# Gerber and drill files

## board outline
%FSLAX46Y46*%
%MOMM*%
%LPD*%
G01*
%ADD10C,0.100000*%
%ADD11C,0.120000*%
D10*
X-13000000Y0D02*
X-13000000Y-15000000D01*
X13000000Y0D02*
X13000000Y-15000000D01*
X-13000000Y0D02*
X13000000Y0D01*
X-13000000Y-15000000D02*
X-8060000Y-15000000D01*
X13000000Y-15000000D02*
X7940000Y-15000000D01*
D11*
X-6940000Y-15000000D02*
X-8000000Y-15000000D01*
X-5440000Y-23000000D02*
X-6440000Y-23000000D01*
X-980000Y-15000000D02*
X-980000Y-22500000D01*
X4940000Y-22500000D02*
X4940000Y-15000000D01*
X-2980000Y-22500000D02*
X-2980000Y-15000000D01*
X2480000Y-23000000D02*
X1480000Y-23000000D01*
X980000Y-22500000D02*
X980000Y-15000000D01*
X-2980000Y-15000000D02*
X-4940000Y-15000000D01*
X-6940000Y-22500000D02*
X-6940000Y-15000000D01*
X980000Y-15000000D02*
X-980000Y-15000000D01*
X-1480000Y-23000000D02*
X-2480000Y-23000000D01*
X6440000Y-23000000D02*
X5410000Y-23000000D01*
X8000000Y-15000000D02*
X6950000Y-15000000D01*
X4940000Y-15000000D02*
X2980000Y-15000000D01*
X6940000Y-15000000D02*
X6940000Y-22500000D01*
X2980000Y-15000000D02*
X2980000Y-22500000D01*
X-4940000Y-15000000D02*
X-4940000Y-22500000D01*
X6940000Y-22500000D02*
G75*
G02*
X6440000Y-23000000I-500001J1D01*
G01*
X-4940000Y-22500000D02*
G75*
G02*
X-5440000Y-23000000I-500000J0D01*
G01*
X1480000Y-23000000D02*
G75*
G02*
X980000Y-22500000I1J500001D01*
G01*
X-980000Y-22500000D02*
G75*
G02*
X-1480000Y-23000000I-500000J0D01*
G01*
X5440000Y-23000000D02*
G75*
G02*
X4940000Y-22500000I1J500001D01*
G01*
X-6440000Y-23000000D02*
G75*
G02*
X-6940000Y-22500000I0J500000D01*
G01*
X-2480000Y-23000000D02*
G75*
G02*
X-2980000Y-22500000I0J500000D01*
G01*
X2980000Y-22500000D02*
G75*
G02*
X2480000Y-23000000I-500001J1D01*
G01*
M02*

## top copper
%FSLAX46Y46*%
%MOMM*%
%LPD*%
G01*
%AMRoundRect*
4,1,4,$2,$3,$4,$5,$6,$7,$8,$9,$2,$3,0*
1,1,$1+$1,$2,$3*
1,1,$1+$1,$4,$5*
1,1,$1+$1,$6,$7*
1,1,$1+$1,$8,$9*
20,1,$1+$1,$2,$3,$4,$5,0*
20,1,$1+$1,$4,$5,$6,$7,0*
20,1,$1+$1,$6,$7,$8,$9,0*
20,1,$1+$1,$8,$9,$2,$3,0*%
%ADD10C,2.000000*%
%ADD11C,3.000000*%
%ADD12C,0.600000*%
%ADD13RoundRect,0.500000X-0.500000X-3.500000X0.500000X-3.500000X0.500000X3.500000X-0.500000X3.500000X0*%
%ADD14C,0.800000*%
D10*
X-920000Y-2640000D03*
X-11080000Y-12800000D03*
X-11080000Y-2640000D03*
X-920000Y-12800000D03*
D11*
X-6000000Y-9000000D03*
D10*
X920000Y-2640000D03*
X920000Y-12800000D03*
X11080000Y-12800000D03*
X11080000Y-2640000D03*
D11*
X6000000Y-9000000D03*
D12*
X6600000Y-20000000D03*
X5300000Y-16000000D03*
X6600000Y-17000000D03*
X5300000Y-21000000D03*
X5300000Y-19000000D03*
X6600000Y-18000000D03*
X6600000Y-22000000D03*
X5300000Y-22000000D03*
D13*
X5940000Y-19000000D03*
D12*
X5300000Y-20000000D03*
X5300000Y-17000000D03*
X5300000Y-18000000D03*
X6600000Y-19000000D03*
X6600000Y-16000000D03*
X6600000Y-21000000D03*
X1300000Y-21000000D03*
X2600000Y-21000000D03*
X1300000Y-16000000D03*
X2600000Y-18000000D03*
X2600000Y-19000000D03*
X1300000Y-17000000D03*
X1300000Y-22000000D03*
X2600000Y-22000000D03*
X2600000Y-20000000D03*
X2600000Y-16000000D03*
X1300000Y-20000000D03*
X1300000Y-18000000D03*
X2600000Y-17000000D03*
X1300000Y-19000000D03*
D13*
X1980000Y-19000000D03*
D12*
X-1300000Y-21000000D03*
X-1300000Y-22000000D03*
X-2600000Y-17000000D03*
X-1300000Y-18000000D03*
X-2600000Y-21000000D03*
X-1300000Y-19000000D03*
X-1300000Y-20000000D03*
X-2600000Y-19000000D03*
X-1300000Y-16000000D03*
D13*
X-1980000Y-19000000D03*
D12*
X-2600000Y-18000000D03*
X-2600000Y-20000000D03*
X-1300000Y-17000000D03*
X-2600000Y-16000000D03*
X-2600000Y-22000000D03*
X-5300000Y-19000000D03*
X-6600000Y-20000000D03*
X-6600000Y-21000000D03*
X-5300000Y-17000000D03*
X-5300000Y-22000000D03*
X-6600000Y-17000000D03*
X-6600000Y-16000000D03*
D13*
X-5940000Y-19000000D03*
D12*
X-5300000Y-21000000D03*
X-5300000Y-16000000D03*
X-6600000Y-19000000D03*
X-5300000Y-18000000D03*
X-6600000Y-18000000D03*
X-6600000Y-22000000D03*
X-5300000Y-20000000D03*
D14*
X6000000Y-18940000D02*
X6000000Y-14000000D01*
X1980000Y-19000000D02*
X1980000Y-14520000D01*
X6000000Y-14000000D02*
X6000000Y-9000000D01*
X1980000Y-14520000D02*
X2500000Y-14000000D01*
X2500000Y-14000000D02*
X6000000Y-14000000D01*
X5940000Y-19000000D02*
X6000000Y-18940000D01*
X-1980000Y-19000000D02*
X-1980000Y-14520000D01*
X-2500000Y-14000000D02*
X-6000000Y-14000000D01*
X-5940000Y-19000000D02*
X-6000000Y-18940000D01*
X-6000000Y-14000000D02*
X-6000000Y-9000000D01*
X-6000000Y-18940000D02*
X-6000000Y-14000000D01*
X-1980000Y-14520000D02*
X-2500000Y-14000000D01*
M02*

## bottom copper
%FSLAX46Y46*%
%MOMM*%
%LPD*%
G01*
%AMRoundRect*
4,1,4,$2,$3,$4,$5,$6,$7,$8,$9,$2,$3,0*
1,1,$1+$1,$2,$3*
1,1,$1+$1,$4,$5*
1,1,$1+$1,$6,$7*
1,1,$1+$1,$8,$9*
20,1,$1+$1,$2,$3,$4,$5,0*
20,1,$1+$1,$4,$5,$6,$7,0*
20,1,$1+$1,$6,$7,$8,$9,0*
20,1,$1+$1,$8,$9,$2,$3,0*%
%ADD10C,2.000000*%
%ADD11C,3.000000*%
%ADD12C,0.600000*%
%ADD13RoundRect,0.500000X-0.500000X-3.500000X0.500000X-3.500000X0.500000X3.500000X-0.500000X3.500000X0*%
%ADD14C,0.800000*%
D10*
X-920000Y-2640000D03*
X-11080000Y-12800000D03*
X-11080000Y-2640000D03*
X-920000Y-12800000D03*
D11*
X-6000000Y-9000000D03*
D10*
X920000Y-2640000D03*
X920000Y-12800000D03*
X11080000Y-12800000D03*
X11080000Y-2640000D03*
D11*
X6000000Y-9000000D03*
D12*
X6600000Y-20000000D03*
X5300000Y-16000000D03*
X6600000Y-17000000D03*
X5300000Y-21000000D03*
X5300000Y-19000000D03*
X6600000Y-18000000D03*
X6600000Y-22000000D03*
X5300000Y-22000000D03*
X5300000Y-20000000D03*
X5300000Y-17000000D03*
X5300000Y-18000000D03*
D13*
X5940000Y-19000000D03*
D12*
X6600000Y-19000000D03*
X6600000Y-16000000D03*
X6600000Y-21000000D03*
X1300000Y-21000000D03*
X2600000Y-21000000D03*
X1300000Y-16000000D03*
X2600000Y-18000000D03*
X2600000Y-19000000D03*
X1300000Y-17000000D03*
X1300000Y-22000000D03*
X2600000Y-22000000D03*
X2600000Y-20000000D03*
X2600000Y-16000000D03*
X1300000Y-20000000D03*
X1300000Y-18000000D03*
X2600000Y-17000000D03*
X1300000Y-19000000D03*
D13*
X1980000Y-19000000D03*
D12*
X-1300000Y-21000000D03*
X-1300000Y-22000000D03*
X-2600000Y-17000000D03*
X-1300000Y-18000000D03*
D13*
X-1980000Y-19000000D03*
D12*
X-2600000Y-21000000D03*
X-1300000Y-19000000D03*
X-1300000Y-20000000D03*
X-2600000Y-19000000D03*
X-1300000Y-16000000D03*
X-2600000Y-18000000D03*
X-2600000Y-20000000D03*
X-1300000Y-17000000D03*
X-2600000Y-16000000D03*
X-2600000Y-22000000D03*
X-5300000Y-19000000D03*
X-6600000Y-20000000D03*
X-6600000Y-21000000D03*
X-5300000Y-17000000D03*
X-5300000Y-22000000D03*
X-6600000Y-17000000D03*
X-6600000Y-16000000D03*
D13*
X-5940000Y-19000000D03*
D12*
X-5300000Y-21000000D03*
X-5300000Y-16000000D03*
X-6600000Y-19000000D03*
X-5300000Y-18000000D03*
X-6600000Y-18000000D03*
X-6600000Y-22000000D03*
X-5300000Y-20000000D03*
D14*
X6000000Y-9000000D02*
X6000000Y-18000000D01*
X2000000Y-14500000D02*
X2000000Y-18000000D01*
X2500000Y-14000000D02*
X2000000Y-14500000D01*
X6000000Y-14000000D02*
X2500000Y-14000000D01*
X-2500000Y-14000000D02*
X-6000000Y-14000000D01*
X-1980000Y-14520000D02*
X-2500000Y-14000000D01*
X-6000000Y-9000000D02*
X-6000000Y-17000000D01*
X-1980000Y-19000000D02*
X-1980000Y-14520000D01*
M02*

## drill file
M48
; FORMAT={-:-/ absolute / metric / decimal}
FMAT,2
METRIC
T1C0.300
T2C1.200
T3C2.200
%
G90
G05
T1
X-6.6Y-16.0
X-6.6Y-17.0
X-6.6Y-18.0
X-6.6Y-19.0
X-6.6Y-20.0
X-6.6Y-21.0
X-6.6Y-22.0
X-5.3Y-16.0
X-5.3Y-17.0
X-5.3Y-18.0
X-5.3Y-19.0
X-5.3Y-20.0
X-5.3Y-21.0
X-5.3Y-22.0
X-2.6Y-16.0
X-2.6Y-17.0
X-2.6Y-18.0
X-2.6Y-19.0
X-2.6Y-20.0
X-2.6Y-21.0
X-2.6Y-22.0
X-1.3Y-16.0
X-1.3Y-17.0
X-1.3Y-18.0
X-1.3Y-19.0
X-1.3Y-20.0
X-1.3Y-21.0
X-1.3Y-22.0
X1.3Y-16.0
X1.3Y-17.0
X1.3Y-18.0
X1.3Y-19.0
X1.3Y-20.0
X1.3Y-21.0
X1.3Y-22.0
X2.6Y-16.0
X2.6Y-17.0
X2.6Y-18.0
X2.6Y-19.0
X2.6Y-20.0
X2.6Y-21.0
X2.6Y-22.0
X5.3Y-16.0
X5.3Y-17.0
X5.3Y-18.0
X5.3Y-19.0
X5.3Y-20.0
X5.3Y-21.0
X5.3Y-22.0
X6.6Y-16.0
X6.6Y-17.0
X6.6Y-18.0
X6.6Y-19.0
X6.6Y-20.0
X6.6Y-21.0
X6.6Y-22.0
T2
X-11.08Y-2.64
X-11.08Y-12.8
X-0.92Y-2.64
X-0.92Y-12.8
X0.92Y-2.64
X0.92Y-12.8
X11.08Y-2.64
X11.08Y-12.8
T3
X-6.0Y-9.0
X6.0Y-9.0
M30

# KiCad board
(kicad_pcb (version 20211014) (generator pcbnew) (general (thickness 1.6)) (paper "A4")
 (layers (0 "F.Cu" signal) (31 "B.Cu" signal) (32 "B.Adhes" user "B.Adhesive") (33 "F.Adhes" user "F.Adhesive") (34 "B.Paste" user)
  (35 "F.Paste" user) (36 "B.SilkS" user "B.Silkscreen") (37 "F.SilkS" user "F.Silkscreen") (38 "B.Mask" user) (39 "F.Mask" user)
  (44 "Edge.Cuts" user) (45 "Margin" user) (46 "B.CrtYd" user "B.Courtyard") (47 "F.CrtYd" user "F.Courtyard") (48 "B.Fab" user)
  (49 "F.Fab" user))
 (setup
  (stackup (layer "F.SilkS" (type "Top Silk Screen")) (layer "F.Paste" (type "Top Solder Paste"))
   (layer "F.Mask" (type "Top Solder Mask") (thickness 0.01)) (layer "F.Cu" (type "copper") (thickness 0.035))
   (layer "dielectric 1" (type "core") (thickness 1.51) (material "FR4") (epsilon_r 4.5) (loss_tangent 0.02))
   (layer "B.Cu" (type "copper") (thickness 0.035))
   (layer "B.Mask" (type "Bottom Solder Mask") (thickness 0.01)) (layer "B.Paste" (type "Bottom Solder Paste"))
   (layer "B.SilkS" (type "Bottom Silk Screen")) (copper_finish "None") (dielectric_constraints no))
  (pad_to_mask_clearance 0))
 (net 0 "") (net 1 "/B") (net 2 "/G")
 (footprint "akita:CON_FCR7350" (layer "F.Cu") (at -6 9 -90)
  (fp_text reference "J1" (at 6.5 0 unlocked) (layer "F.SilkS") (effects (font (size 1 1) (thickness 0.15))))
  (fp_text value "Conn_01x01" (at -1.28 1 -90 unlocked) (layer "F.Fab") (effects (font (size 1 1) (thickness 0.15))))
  (pad "-" thru_hole circle (at -6.36 -5.08 270) (size 2 2) (drill 1.2) (layers *.Cu *.Mask))
  (pad "-" thru_hole circle (at 3.8 5.08 270) (size 2 2) (drill 1.2) (layers *.Cu *.Mask))
  (pad "-" thru_hole circle (at -6.36 5.08 270) (size 2 2) (drill 1.2) (layers *.Cu *.Mask))
  (pad "-" thru_hole circle (at 3.8 -5.08 270) (size 2 2) (drill 1.2) (layers *.Cu *.Mask))
  (pad "1" thru_hole circle (at 0 0 270) (size 3 3) (drill 2.2) (layers *.Cu *.Mask) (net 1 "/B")))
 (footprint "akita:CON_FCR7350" (layer "F.Cu") (at 6 9 -90)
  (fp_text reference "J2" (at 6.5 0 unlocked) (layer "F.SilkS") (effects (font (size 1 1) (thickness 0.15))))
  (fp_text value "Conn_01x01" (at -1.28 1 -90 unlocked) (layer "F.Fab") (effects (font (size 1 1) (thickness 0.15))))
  (pad "-" thru_hole circle (at -6.36 5.08 270) (size 2 2) (drill 1.2) (layers *.Cu *.Mask))
  (pad "-" thru_hole circle (at 3.8 5.08 270) (size 2 2) (drill 1.2) (layers *.Cu *.Mask))
  (pad "-" thru_hole circle (at 3.8 -5.08 270) (size 2 2) (drill 1.2) (layers *.Cu *.Mask))
  (pad "-" thru_hole circle (at -6.36 -5.08 270) (size 2 2) (drill 1.2) (layers *.Cu *.Mask))
  (pad "1" thru_hole circle (at 0 0 270) (size 3 3) (drill 2.2) (layers *.Cu *.Mask) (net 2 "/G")))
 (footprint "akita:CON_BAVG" (layer "F.Cu") (at 0 19 180)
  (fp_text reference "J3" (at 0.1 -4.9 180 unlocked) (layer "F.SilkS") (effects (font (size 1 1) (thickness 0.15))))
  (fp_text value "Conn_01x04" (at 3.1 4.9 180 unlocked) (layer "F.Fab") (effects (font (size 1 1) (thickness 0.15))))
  (fp_line (start 6.94 4) (end 8 4) (layer "Edge.Cuts") (width 0.12))
  (fp_line (start 5.44 -4) (end 6.44 -4) (layer "Edge.Cuts") (width 0.12))
  (fp_line (start 0.98 4) (end 0.98 -3.5) (layer "Edge.Cuts") (width 0.12))
  (fp_line (start -4.94 -3.5) (end -4.94 4) (layer "Edge.Cuts") (width 0.12))
  (fp_line (start 2.98 -3.5) (end 2.98 4) (layer "Edge.Cuts") (width 0.12))
  (fp_line (start -2.48 -4) (end -1.48 -4) (layer "Edge.Cuts") (width 0.12))
  (fp_line (start -0.98 -3.5) (end -0.98 4) (layer "Edge.Cuts") (width 0.12))
  (fp_line (start 2.98 4) (end 4.94 4) (layer "Edge.Cuts") (width 0.12))
  (fp_line (start 6.94 -3.5) (end 6.94 4) (layer "Edge.Cuts") (width 0.12))
  (fp_line (start -0.98 4) (end 0.98 4) (layer "Edge.Cuts") (width 0.12))
  (fp_line (start 1.48 -4) (end 2.48 -4) (layer "Edge.Cuts") (width 0.12))
  (fp_line (start -6.44 -4) (end -5.41 -4) (layer "Edge.Cuts") (width 0.12))
  (fp_line (start -8 4) (end -6.95 4) (layer "Edge.Cuts") (width 0.12))
  (fp_line (start -4.94 4) (end -2.98 4) (layer "Edge.Cuts") (width 0.12))
  (fp_line (start -6.94 4) (end -6.94 -3.5) (layer "Edge.Cuts") (width 0.12))
  (fp_line (start -2.98 4) (end -2.98 -3.5) (layer "Edge.Cuts") (width 0.12))
  (fp_line (start 4.94 4) (end 4.94 -3.5) (layer "Edge.Cuts") (width 0.12))
  (fp_arc (start -6.94 -3.5) (mid -6.793553 -3.853553) (end -6.44 -4) (layer "Edge.Cuts") (width 0.12))
  (fp_arc (start 4.94 -3.5) (mid 5.086447 -3.853553) (end 5.44 -4) (layer "Edge.Cuts") (width 0.12))
  (fp_arc (start -1.48 -4) (mid -1.126447 -3.853553) (end -0.98 -3.5) (layer "Edge.Cuts") (width 0.12))
  (fp_arc (start 0.98 -3.5) (mid 1.126447 -3.853553) (end 1.48 -4) (layer "Edge.Cuts") (width 0.12))
  (fp_arc (start -5.44 -4) (mid -5.086447 -3.853553) (end -4.94 -3.5) (layer "Edge.Cuts") (width 0.12))
  (fp_arc (start 6.44 -4) (mid 6.793553 -3.853553) (end 6.94 -3.5) (layer "Edge.Cuts") (width 0.12))
  (fp_arc (start 2.48 -4) (mid 2.833553 -3.853553) (end 2.98 -3.5) (layer "Edge.Cuts") (width 0.12))
  (fp_arc (start -2.98 -3.5) (mid -2.833553 -3.853553) (end -2.48 -4) (layer "Edge.Cuts") (width 0.12))
  (pad "1" thru_hole circle (at -6.6 -1 180) (size 0.6 0.6) (drill 0.3) (layers *.Cu *.Mask) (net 2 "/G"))
  (pad "1" thru_hole circle (at -5.3 3 180) (size 0.6 0.6) (drill 0.3) (layers *.Cu *.Mask) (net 2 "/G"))
  (pad "1" thru_hole circle (at -6.6 2 180) (size 0.6 0.6) (drill 0.3) (layers *.Cu *.Mask) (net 2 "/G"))
  (pad "1" thru_hole circle (at -5.3 -2 180) (size 0.6 0.6) (drill 0.3) (layers *.Cu *.Mask) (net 2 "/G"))
  (pad "1" thru_hole circle (at -5.3 0 180) (size 0.6 0.6) (drill 0.3) (layers *.Cu *.Mask) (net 2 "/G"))
  (pad "1" thru_hole circle (at -6.6 1 180) (size 0.6 0.6) (drill 0.3) (layers *.Cu *.Mask) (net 2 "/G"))
  (pad "1" thru_hole circle (at -6.6 -3 180) (size 0.6 0.6) (drill 0.3) (layers *.Cu *.Mask) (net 2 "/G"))
  (pad "1" thru_hole circle (at -5.3 -3 180) (size 0.6 0.6) (drill 0.3) (layers *.Cu *.Mask) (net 2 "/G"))
  (pad "1" smd roundrect (at -5.94 0) (size 2 8) (layers "F.Cu" "F.Paste" "F.Mask") (roundrect_rratio 0.25) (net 2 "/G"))
  (pad "1" thru_hole circle (at -5.3 -1 180) (size 0.6 0.6) (drill 0.3) (layers *.Cu *.Mask) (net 2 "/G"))
  (pad "1" thru_hole circle (at -5.3 2 180) (size 0.6 0.6) (drill 0.3) (layers *.Cu *.Mask) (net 2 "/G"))
  (pad "1" thru_hole circle (at -5.3 1 180) (size 0.6 0.6) (drill 0.3) (layers *.Cu *.Mask) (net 2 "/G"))
  (pad "1" smd roundrect (at -5.94 0) (size 2 8) (layers "B.Cu" "B.Paste" "B.Mask") (roundrect_rratio 0.25) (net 2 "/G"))
  (pad "1" thru_hole circle (at -6.6 0 180) (size 0.6 0.6) (drill 0.3) (layers *.Cu *.Mask) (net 2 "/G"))
  (pad "1" thru_hole circle (at -6.6 3 180) (size 0.6 0.6) (drill 0.3) (layers *.Cu *.Mask) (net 2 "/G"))
  (pad "1" thru_hole circle (at -6.6 -2 180) (size 0.6 0.6) (drill 0.3) (layers *.Cu *.Mask) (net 2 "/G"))
  (pad "2" thru_hole circle (at -1.3 -2 180) (size 0.6 0.6) (drill 0.3) (layers *.Cu *.Mask) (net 2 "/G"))
  (pad "2" thru_hole circle (at -2.6 -2 180) (size 0.6 0.6) (drill 0.3) (layers *.Cu *.Mask) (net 2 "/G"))
  (pad "2" thru_hole circle (at -1.3 3 180) (size 0.6 0.6) (drill 0.3) (layers *.Cu *.Mask) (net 2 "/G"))
  (pad "2" thru_hole circle (at -2.6 1 180) (size 0.6 0.6) (drill 0.3) (layers *.Cu *.Mask) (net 2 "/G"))
  (pad "2" thru_hole circle (at -2.6 0 180) (size 0.6 0.6) (drill 0.3) (layers *.Cu *.Mask) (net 2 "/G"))
  (pad "2" thru_hole circle (at -1.3 2 180) (size 0.6 0.6) (drill 0.3) (layers *.Cu *.Mask) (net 2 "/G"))
  (pad "2" thru_hole circle (at -1.3 -3 180) (size 0.6 0.6) (drill 0.3) (layers *.Cu *.Mask) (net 2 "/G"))
  (pad "2" thru_hole circle (at -2.6 -3 180) (size 0.6 0.6) (drill 0.3) (layers *.Cu *.Mask) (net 2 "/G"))
  (pad "2" thru_hole circle (at -2.6 -1 180) (size 0.6 0.6) (drill 0.3) (layers *.Cu *.Mask) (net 2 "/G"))
  (pad "2" thru_hole circle (at -2.6 3 180) (size 0.6 0.6) (drill 0.3) (layers *.Cu *.Mask) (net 2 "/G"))
  (pad "2" thru_hole circle (at -1.3 -1 180) (size 0.6 0.6) (drill 0.3) (layers *.Cu *.Mask) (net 2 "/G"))
  (pad "2" thru_hole circle (at -1.3 1 180) (size 0.6 0.6) (drill 0.3) (layers *.Cu *.Mask) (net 2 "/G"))
  (pad "2" thru_hole circle (at -2.6 2 180) (size 0.6 0.6) (drill 0.3) (layers *.Cu *.Mask) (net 2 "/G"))
  (pad "2" thru_hole circle (at -1.3 0 180) (size 0.6 0.6) (drill 0.3) (layers *.Cu *.Mask) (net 2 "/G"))
  (pad "2" smd roundrect (at -1.98 0) (size 2 8) (layers "F.Cu" "F.Paste" "F.Mask") (roundrect_rratio 0.25) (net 2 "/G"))
  (pad "2" smd roundrect (at -1.98 0) (size 2 8) (layers "B.Cu" "B.Paste" "B.Mask") (roundrect_rratio 0.25) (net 2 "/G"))
  (pad "3" thru_hole circle (at 1.3 -2 180) (size 0.6 0.6) (drill 0.3) (layers *.Cu *.Mask) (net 1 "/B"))
  (pad "3" thru_hole circle (at 1.3 -3 180) (size 0.6 0.6) (drill 0.3) (layers *.Cu *.Mask) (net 1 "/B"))
  (pad "3" thru_hole circle (at 2.6 2 180) (size 0.6 0.6) (drill 0.3) (layers *.Cu *.Mask) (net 1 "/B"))
  (pad "3" thru_hole circle (at 1.3 1 180) (size 0.6 0.6) (drill 0.3) (layers *.Cu *.Mask) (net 1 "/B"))
  (pad "3" smd roundrect (at 1.98 0) (size 2 8) (layers "B.Cu" "B.Paste" "B.Mask") (roundrect_rratio 0.25) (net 1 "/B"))
  (pad "3" thru_hole circle (at 2.6 -2 180) (size 0.6 0.6) (drill 0.3) (layers *.Cu *.Mask) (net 1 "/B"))
  (pad "3" thru_hole circle (at 1.3 0 180) (size 0.6 0.6) (drill 0.3) (layers *.Cu *.Mask) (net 1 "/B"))
  (pad "3" thru_hole circle (at 1.3 -1 180) (size 0.6 0.6) (drill 0.3) (layers *.Cu *.Mask) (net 1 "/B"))
  (pad "3" thru_hole circle (at 2.6 0 180) (size 0.6 0.6) (drill 0.3) (layers *.Cu *.Mask) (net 1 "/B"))
  (pad "3" thru_hole circle (at 1.3 3 180) (size 0.6 0.6) (drill 0.3) (layers *.Cu *.Mask) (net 1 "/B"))
  (pad "3" smd roundrect (at 1.98 0) (size 2 8) (layers "F.Cu" "F.Paste" "F.Mask") (roundrect_rratio 0.25) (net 1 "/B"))
  (pad "3" thru_hole circle (at 2.6 1 180) (size 0.6 0.6) (drill 0.3) (layers *.Cu *.Mask) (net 1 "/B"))
  (pad "3" thru_hole circle (at 2.6 -1 180) (size 0.6 0.6) (drill 0.3) (layers *.Cu *.Mask) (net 1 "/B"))
  (pad "3" thru_hole circle (at 1.3 2 180) (size 0.6 0.6) (drill 0.3) (layers *.Cu *.Mask) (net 1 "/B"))
  (pad "3" thru_hole circle (at 2.6 3 180) (size 0.6 0.6) (drill 0.3) (layers *.Cu *.Mask) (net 1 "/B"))
  (pad "3" thru_hole circle (at 2.6 -3 180) (size 0.6 0.6) (drill 0.3) (layers *.Cu *.Mask) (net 1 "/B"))
  (pad "4" thru_hole circle (at 5.3 0 180) (size 0.6 0.6) (drill 0.3) (layers *.Cu *.Mask) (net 1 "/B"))
  (pad "4" thru_hole circle (at 6.6 -1 180) (size 0.6 0.6) (drill 0.3) (layers *.Cu *.Mask) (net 1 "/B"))
  (pad "4" thru_hole circle (at 6.6 -2 180) (size 0.6 0.6) (drill 0.3) (layers *.Cu *.Mask) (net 1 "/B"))
  (pad "4" thru_hole circle (at 5.3 2 180) (size 0.6 0.6) (drill 0.3) (layers *.Cu *.Mask) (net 1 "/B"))
  (pad "4" thru_hole circle (at 5.3 -3 180) (size 0.6 0.6) (drill 0.3) (layers *.Cu *.Mask) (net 1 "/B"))
  (pad "4" thru_hole circle (at 6.6 2 180) (size 0.6 0.6) (drill 0.3) (layers *.Cu *.Mask) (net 1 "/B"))
  (pad "4" thru_hole circle (at 6.6 3 180) (size 0.6 0.6) (drill 0.3) (layers *.Cu *.Mask) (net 1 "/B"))
  (pad "4" smd roundrect (at 5.94 0) (size 2 8) (layers "F.Cu" "F.Paste" "F.Mask") (roundrect_rratio 0.25) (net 1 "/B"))
  (pad "4" smd roundrect (at 5.94 0) (size 2 8) (layers "B.Cu" "B.Paste" "B.Mask") (roundrect_rratio 0.25) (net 1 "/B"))
  (pad "4" thru_hole circle (at 5.3 -2 180) (size 0.6 0.6) (drill 0.3) (layers *.Cu *.Mask) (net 1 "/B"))
  (pad "4" thru_hole circle (at 5.3 3 180) (size 0.6 0.6) (drill 0.3) (layers *.Cu *.Mask) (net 1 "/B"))
  (pad "4" thru_hole circle (at 6.6 0 180) (size 0.6 0.6) (drill 0.3) (layers *.Cu *.Mask) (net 1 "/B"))
  (pad "4" thru_hole circle (at 5.3 1 180) (size 0.6 0.6) (drill 0.3) (layers *.Cu *.Mask) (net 1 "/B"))
  (pad "4" thru_hole circle (at 6.6 1 180) (size 0.6 0.6) (drill 0.3) (layers *.Cu *.Mask) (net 1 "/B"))
  (pad "4" thru_hole circle (at 6.6 -3 180) (size 0.6 0.6) (drill 0.3) (layers *.Cu *.Mask) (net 1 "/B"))
  (pad "4" thru_hole circle (at 5.3 -1 180) (size 0.6 0.6) (drill 0.3) (layers *.Cu *.Mask) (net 1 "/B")))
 (gr_line (start -13 0) (end -13 15) (layer "Edge.Cuts") (width 0.1))
 (gr_line (start 13 0) (end 13 15) (layer "Edge.Cuts") (width 0.1))
 (gr_line (start -13 0) (end 13 0) (layer "Edge.Cuts") (width 0.1))
 (gr_line (start -13 15) (end -8.06 15) (layer "Edge.Cuts") (width 0.1))
 (gr_line (start 13 15) (end 7.94 15) (layer "Edge.Cuts") (width 0.1))
 (segment (start 6 18.94) (end 6 14) (width 0.8) (layer "F.Cu") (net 2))
 (segment (start 1.98 19) (end 1.98 14.52) (width 0.8) (layer "F.Cu") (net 2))
 (segment (start 6 14) (end 6 9) (width 0.8) (layer "F.Cu") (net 2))
 (segment (start 1.98 14.52) (end 2.5 14) (width 0.8) (layer "F.Cu") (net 2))
 (segment (start 2.5 14) (end 6 14) (width 0.8) (layer "F.Cu") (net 2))
 (segment (start 5.94 19) (end 6 18.94) (width 0.8) (layer "F.Cu") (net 2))
 (segment (start 6 9) (end 6 18) (width 0.8) (layer "B.Cu") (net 2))
 (segment (start 2 14.5) (end 2 18) (width 0.8) (layer "B.Cu") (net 2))
 (segment (start 2.5 14) (end 2 14.5) (width 0.8) (layer "B.Cu") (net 2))
 (segment (start 6 14) (end 2.5 14) (width 0.8) (layer "B.Cu") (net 2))
 (segment (start -1.98 19) (end -1.98 14.52) (width 0.8) (layer "F.Cu") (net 1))
 (segment (start -2.5 14) (end -6 14) (width 0.8) (layer "F.Cu") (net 1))
 (segment (start -5.94 19) (end -6 18.94) (width 0.8) (layer "F.Cu") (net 1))
 (segment (start -6 14) (end -6 9) (width 0.8) (layer "F.Cu") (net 1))
 (segment (start -6 18.94) (end -6 14) (width 0.8) (layer "F.Cu") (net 1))
 (segment (start -1.98 14.52) (end -2.5 14) (width 0.8) (layer "F.Cu") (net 1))
 (segment (start -2.5 14) (end -6 14) (width 0.8) (layer "B.Cu") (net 1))
 (segment (start -1.98 14.52) (end -2.5 14) (width 0.8) (layer "B.Cu") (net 1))
 (segment (start -6 9) (end -6 17) (width 0.8) (layer "B.Cu") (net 1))
 (segment (start -1.98 19) (end -1.98 14.52) (width 0.8) (layer "B.Cu") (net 1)))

